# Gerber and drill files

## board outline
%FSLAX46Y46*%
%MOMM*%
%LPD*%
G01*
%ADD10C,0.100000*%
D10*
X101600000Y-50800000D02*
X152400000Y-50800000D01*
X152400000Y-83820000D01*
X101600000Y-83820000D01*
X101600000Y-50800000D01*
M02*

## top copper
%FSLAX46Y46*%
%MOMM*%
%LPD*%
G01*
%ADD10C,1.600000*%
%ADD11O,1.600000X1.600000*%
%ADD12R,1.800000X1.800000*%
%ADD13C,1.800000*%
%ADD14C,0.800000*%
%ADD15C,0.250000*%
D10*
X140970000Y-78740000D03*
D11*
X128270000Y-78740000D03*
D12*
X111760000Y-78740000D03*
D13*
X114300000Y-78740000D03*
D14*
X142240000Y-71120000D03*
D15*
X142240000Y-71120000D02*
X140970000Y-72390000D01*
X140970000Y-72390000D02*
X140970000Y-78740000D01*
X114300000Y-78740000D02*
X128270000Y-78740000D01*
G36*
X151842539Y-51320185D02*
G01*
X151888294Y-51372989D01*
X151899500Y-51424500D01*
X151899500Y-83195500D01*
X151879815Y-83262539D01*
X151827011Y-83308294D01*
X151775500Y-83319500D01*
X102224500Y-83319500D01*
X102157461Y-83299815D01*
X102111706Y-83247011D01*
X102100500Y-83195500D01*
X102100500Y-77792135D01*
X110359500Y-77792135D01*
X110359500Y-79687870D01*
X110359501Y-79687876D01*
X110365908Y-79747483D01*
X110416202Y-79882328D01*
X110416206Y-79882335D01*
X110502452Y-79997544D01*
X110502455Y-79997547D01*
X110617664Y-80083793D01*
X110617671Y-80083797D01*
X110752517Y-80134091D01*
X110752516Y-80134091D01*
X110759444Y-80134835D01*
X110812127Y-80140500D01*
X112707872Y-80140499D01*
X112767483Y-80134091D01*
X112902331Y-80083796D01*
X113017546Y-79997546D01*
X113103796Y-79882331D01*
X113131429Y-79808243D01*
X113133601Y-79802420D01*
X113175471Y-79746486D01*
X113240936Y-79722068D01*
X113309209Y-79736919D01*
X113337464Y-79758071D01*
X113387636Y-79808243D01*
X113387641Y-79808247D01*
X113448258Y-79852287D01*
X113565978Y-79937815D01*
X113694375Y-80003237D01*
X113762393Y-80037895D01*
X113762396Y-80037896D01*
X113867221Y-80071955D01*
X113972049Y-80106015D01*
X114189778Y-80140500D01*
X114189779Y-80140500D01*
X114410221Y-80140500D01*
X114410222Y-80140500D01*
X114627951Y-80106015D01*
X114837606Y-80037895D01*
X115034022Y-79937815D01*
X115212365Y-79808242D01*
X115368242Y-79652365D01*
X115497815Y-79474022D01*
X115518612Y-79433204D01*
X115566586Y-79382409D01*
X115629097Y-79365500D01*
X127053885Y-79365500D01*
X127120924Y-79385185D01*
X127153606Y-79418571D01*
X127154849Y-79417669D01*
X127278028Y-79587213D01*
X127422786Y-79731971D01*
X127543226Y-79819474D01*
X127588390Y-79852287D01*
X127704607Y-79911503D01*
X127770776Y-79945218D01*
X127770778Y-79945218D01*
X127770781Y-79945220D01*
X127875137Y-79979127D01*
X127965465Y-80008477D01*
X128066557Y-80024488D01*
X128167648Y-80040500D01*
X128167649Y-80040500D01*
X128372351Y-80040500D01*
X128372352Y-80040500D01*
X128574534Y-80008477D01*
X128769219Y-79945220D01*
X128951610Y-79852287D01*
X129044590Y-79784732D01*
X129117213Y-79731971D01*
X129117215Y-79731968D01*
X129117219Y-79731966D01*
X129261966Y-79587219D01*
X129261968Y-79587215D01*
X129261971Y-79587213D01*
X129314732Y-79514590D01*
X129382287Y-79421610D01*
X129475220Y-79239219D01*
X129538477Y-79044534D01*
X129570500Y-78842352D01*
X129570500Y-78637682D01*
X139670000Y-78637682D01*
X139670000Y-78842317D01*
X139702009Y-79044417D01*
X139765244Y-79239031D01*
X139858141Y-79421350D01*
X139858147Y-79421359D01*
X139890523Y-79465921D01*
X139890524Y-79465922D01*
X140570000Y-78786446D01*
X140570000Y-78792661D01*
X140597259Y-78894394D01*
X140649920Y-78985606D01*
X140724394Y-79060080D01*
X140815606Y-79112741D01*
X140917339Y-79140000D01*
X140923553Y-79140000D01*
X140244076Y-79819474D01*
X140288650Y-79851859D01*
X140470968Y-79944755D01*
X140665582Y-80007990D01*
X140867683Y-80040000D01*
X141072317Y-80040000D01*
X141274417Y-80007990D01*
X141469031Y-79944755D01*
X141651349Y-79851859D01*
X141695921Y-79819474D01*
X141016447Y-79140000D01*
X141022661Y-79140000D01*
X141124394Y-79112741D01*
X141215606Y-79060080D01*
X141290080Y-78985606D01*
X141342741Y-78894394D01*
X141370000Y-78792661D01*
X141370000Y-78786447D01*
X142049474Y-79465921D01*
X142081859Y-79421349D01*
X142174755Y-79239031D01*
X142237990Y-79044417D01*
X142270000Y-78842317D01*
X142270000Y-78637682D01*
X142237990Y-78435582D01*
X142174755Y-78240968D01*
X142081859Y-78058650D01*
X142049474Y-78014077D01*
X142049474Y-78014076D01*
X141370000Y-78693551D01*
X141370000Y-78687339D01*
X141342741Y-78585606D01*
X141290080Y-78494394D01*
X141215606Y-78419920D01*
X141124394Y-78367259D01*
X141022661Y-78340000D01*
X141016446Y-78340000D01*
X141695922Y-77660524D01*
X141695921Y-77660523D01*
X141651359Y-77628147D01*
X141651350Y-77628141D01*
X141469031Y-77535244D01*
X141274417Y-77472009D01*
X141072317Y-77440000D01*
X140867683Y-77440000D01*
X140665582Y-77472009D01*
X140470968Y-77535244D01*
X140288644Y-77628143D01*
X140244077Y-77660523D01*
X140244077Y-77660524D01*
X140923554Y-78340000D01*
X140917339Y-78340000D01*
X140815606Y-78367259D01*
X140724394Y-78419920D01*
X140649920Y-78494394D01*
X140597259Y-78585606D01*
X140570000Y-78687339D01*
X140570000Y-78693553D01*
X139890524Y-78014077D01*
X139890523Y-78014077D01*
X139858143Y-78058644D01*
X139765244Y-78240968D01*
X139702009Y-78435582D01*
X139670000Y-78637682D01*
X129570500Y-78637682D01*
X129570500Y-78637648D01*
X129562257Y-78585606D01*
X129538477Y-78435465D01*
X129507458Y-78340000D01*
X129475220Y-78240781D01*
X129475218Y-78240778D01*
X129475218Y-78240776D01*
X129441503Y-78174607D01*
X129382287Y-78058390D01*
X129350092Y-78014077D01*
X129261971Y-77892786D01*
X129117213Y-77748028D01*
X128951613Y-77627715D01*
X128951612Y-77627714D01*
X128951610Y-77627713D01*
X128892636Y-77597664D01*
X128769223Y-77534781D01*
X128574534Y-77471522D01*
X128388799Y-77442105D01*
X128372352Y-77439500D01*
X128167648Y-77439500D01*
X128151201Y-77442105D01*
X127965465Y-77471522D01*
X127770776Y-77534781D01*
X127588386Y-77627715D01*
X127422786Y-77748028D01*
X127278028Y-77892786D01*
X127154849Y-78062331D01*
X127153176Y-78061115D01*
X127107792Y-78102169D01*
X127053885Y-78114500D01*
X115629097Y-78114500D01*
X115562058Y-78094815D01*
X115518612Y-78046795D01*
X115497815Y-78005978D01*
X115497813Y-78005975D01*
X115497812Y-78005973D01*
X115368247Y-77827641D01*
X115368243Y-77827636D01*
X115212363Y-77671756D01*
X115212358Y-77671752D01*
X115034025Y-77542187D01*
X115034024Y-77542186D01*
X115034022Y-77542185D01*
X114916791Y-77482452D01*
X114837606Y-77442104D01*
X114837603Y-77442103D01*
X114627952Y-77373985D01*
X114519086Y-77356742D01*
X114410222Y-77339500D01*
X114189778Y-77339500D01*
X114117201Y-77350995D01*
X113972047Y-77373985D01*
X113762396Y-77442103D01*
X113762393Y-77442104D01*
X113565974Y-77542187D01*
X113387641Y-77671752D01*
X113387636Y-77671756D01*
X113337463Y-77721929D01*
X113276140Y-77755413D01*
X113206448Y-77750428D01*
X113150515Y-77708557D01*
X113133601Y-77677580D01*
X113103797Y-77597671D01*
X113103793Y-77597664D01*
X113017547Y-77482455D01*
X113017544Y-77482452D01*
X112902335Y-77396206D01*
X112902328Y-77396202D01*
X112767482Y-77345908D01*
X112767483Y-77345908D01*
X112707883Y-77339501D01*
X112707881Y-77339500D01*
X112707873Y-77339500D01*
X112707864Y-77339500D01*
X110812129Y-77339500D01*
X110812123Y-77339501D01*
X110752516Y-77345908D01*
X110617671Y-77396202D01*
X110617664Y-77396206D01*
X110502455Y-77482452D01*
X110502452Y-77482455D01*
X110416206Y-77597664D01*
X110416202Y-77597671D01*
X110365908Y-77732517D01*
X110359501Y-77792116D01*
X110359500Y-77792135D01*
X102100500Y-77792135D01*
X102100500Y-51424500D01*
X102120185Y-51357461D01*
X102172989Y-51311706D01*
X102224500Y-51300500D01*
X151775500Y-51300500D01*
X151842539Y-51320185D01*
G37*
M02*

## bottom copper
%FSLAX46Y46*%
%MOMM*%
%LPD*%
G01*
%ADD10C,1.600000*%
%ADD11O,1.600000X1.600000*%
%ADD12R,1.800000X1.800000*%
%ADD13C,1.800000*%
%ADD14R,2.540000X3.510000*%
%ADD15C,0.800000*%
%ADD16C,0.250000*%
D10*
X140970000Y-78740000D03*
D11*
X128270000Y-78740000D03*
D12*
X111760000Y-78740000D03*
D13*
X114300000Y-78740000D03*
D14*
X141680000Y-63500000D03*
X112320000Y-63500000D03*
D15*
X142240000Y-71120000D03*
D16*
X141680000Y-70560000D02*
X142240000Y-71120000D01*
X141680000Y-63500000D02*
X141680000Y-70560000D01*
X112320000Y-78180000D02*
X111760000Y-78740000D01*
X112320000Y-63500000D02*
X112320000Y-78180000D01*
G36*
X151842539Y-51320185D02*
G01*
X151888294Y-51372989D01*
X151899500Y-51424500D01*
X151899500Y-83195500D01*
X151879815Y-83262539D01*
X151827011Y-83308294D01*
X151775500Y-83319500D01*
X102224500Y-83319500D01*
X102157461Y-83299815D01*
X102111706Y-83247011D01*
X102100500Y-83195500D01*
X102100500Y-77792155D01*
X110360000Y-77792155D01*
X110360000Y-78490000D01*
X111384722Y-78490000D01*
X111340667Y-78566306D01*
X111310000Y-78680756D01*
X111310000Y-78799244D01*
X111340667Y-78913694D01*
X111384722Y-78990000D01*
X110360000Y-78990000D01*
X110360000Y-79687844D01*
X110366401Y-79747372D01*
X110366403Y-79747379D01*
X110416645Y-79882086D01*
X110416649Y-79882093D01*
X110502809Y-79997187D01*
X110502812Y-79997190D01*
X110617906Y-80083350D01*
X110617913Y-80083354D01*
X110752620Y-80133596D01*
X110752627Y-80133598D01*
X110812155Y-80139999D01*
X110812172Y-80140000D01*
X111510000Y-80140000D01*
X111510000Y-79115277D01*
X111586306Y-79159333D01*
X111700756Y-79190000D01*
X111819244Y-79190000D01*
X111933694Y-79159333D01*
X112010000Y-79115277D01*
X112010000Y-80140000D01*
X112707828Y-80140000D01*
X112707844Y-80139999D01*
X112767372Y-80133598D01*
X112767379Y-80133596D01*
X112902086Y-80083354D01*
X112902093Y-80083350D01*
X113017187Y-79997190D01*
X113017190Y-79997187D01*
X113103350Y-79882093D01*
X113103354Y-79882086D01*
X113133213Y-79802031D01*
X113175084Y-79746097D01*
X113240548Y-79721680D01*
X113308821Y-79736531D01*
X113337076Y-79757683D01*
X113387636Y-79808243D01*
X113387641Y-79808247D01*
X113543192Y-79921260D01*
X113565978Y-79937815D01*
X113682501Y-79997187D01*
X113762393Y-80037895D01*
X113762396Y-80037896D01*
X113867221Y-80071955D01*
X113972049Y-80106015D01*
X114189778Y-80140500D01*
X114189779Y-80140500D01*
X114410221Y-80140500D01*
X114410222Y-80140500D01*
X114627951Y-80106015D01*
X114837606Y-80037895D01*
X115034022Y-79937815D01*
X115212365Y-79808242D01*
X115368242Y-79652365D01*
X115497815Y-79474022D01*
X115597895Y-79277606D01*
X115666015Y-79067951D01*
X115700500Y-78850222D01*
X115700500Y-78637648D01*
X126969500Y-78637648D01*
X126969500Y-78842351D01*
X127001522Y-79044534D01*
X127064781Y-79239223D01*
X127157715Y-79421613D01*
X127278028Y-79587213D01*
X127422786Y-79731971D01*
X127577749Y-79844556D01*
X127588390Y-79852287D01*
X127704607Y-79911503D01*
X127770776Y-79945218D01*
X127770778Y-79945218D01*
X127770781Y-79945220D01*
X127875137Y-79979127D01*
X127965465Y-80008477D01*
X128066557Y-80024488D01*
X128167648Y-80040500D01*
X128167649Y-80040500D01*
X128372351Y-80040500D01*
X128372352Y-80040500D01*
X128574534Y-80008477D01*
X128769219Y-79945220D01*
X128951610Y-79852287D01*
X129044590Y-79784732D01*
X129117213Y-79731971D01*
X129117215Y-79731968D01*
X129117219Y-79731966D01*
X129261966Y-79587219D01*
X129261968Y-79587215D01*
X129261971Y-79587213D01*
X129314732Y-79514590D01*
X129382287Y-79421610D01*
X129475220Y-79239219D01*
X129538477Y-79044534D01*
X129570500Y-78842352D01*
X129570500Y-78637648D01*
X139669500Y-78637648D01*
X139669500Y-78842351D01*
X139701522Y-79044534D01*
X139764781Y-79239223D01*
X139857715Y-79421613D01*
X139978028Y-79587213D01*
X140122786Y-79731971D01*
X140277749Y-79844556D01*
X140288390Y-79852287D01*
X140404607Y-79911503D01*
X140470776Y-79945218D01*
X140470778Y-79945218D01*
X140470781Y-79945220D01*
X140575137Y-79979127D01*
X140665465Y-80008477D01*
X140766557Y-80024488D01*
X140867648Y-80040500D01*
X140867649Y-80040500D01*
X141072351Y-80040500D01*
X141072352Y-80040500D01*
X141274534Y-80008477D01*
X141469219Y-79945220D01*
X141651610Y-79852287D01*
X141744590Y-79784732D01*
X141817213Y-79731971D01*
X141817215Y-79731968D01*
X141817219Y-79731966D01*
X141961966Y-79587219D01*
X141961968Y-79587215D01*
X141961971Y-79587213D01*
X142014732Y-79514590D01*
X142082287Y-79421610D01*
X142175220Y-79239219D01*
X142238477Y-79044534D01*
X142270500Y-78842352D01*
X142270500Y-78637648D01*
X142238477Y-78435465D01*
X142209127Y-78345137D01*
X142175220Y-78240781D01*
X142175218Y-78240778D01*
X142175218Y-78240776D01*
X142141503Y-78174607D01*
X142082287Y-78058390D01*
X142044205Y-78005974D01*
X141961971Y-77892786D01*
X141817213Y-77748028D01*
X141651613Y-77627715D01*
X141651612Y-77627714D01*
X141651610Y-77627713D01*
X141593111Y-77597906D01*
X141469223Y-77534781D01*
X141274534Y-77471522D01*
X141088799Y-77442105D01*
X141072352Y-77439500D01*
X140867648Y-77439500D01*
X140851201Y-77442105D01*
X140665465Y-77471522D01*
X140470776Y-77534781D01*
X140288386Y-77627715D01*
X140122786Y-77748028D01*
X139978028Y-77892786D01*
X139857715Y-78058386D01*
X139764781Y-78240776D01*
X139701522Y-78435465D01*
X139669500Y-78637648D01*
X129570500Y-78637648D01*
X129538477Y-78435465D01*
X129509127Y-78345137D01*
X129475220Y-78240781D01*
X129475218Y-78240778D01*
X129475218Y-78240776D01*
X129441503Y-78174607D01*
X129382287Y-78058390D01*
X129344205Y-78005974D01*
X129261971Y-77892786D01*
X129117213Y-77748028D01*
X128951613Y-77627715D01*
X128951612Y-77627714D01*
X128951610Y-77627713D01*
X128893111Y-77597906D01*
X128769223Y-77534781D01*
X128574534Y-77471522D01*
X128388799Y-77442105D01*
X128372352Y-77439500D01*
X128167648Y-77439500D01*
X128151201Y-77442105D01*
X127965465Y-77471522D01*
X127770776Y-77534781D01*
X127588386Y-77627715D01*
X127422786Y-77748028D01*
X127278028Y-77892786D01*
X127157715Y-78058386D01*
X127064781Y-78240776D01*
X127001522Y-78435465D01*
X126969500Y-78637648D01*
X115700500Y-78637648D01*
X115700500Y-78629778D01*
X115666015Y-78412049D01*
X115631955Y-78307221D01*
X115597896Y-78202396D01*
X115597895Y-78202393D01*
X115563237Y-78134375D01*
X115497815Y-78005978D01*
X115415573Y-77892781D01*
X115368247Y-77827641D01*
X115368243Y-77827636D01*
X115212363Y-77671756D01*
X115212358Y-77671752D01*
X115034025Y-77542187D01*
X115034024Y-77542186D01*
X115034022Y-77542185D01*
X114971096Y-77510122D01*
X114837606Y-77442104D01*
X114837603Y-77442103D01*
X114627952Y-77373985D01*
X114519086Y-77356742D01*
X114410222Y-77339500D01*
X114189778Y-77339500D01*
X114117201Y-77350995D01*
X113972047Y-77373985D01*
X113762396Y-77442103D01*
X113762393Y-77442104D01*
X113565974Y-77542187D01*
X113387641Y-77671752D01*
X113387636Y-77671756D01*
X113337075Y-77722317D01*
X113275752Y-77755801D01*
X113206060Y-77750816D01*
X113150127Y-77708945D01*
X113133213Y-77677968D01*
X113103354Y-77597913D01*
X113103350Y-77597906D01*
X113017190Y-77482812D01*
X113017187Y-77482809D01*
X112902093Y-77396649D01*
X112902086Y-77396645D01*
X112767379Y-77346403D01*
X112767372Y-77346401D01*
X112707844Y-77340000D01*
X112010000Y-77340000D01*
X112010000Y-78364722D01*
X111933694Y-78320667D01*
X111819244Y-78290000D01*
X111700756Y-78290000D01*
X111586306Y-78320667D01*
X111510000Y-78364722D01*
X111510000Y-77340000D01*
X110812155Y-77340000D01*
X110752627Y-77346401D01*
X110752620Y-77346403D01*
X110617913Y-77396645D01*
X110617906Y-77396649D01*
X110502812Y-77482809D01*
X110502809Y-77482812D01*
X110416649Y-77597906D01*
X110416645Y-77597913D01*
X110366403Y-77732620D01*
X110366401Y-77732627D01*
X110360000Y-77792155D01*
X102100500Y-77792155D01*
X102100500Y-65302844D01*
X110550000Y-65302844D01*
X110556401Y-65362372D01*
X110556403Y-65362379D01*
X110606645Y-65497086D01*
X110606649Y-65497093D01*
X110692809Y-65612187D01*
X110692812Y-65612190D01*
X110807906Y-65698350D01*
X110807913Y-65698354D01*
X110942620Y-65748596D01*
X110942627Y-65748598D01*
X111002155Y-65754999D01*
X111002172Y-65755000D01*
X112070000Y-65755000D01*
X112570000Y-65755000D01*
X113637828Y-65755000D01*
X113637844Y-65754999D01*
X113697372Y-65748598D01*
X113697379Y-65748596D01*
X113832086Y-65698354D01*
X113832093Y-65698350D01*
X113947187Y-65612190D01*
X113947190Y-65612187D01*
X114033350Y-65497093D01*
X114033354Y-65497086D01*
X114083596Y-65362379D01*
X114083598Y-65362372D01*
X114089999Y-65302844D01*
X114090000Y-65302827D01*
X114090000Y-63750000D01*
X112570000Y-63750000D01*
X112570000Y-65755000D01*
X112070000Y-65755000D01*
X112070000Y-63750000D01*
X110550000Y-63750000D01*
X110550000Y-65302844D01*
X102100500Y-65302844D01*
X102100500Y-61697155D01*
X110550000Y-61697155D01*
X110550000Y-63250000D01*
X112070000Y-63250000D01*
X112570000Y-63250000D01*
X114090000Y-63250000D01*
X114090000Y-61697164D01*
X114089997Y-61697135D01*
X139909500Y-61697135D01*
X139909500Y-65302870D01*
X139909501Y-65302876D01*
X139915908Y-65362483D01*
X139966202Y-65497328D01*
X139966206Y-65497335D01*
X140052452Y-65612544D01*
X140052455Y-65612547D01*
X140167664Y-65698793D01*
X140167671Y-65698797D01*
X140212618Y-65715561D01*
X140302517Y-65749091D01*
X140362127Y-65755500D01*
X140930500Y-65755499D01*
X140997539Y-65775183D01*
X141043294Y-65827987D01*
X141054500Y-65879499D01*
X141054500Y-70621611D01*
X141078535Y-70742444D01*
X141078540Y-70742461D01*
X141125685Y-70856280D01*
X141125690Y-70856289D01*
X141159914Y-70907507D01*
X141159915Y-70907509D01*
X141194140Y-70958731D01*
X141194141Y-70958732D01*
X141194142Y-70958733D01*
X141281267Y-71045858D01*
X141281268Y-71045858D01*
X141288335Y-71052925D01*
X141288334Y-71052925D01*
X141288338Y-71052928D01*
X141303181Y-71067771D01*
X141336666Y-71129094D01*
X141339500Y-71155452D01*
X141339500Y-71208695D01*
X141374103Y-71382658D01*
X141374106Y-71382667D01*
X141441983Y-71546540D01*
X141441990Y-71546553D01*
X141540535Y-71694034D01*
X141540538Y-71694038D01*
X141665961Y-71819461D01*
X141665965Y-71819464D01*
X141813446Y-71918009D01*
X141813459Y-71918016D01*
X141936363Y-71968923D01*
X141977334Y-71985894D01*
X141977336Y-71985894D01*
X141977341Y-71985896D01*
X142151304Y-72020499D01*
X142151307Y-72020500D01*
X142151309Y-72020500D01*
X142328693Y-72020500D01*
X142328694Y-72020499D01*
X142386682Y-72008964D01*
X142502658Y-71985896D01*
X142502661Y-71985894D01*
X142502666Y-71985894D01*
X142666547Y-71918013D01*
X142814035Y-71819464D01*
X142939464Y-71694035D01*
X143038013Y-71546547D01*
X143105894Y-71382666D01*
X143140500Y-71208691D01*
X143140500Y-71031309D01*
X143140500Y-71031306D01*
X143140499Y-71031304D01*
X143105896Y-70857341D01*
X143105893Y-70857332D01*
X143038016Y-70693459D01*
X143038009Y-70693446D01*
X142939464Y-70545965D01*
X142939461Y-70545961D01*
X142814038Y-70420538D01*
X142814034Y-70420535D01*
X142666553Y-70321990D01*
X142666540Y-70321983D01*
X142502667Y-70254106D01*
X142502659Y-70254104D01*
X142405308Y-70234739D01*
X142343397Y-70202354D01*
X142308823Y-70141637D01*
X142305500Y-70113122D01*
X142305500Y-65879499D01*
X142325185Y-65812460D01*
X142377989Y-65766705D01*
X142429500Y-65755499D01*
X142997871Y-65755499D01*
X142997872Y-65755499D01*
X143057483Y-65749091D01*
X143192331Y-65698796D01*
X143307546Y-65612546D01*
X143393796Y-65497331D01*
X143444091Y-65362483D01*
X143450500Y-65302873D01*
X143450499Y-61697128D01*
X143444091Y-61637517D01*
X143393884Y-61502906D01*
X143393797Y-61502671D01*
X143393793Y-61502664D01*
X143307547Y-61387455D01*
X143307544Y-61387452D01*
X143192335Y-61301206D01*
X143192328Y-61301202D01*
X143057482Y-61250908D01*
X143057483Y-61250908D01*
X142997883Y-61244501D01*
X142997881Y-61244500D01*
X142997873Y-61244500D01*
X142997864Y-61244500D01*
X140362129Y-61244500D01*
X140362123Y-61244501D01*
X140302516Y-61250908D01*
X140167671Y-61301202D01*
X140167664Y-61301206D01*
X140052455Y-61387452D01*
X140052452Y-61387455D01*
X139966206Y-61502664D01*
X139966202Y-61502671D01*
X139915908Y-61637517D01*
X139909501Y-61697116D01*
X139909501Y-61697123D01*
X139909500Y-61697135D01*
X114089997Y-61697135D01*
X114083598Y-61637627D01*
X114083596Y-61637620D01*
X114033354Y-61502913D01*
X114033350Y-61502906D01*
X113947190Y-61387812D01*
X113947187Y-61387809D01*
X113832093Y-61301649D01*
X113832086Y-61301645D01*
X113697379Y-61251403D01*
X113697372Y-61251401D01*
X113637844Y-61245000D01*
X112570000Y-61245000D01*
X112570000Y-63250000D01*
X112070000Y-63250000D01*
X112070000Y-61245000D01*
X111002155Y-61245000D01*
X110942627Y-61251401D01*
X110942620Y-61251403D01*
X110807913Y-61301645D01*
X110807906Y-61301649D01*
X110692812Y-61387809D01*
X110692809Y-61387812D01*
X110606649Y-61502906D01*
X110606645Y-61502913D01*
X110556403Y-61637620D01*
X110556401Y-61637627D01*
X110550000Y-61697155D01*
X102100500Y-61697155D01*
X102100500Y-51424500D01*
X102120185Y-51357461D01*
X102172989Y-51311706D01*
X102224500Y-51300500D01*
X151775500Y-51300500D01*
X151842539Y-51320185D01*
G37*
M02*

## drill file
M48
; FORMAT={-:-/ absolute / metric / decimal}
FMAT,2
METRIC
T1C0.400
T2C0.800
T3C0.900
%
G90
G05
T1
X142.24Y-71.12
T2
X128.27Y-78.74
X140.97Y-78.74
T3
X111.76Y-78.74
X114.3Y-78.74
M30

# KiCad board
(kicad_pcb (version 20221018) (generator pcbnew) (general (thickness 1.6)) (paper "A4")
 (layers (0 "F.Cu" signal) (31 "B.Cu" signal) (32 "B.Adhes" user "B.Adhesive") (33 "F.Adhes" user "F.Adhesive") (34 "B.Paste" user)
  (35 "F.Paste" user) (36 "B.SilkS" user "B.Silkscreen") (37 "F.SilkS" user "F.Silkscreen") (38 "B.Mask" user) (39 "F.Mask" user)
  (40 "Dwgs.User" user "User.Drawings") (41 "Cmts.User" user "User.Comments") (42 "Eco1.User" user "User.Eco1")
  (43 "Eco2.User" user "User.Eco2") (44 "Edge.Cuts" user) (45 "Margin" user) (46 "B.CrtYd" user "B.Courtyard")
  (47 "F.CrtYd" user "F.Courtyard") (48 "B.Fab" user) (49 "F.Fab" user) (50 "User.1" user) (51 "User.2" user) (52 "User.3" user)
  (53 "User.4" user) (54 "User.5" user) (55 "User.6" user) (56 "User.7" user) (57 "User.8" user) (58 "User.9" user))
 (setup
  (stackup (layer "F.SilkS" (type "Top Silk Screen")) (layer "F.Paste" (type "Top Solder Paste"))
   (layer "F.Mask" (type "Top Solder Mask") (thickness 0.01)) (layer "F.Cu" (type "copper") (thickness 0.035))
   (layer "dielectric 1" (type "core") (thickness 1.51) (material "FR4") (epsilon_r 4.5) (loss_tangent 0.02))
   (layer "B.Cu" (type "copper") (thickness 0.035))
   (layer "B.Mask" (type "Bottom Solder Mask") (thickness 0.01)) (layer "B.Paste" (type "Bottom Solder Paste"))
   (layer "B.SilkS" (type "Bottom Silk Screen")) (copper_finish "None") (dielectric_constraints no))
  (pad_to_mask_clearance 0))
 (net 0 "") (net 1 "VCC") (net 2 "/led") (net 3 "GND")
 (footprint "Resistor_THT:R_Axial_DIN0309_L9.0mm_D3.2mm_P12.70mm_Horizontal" (layer "F.Cu") (at 140.97 78.74 180)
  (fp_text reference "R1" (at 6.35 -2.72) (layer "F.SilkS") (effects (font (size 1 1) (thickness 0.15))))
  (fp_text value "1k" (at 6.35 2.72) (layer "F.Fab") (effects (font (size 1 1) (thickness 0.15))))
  (pad "1" thru_hole circle (at 0 0 180) (size 1.6 1.6) (drill 0.8) (layers "*.Cu" "*.Mask") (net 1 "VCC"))
  (pad "2" thru_hole oval (at 12.7 0 180) (size 1.6 1.6) (drill 0.8) (layers "*.Cu" "*.Mask") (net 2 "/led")))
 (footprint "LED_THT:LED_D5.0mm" (layer "F.Cu") (at 111.76 78.74)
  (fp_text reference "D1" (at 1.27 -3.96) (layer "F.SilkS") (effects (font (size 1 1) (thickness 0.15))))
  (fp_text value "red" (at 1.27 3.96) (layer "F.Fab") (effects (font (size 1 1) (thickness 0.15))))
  (pad "1" thru_hole rect (at 0 0) (size 1.8 1.8) (drill 0.9) (layers "*.Cu" "*.Mask") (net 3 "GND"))
  (pad "2" thru_hole circle (at 2.54 0) (size 1.8 1.8) (drill 0.9) (layers "*.Cu" "*.Mask") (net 2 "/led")))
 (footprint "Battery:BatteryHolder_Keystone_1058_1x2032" (layer "B.Cu") (at 127 63.5 180)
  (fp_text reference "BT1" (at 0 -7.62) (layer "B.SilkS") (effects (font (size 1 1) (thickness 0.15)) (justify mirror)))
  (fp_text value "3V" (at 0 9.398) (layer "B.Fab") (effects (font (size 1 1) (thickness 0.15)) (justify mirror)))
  (pad "1" smd rect (at -14.68 0 180) (size 2.54 3.51) (layers "B.Cu" "B.Paste" "B.Mask") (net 1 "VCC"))
  (pad "2" smd rect (at 14.68 0 180) (size 2.54 3.51) (layers "B.Cu" "B.Paste" "B.Mask") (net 3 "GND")))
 (gr_rect (start 101.6 50.8) (end 152.4 83.82) (stroke (width 0.1) (type default)) (fill none) (layer "Edge.Cuts"))
 (segment (start 142.24 71.12) (end 140.97 72.39) (width 0.25) (layer "F.Cu") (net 1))
 (segment (start 140.97 72.39) (end 140.97 78.74) (width 0.25) (layer "F.Cu") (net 1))
 (via (at 142.24 71.12) (size 0.8) (drill 0.4) (layers "F.Cu" "B.Cu") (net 1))
 (segment (start 141.68 70.56) (end 142.24 71.12) (width 0.25) (layer "B.Cu") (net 1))
 (segment (start 141.68 63.5) (end 141.68 70.56) (width 0.25) (layer "B.Cu") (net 1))
 (segment (start 112.32 78.18) (end 111.76 78.74) (width 0.25) (layer "B.Cu") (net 3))
 (segment (start 112.32 63.5) (end 112.32 78.18) (width 0.25) (layer "B.Cu") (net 3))
 (segment (start 114.3 78.74) (end 128.27 78.74) (width 0.25) (layer "F.Cu") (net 2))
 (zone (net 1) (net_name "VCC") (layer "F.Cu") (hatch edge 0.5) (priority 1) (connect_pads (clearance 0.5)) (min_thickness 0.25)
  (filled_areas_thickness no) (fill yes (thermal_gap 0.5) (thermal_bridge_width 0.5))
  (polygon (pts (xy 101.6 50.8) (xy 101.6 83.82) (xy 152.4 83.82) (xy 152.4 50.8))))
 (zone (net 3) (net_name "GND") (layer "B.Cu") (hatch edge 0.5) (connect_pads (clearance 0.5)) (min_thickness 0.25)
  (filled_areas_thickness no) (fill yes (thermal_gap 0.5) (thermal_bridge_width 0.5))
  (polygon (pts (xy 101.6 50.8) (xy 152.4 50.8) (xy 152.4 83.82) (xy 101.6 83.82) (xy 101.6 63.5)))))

